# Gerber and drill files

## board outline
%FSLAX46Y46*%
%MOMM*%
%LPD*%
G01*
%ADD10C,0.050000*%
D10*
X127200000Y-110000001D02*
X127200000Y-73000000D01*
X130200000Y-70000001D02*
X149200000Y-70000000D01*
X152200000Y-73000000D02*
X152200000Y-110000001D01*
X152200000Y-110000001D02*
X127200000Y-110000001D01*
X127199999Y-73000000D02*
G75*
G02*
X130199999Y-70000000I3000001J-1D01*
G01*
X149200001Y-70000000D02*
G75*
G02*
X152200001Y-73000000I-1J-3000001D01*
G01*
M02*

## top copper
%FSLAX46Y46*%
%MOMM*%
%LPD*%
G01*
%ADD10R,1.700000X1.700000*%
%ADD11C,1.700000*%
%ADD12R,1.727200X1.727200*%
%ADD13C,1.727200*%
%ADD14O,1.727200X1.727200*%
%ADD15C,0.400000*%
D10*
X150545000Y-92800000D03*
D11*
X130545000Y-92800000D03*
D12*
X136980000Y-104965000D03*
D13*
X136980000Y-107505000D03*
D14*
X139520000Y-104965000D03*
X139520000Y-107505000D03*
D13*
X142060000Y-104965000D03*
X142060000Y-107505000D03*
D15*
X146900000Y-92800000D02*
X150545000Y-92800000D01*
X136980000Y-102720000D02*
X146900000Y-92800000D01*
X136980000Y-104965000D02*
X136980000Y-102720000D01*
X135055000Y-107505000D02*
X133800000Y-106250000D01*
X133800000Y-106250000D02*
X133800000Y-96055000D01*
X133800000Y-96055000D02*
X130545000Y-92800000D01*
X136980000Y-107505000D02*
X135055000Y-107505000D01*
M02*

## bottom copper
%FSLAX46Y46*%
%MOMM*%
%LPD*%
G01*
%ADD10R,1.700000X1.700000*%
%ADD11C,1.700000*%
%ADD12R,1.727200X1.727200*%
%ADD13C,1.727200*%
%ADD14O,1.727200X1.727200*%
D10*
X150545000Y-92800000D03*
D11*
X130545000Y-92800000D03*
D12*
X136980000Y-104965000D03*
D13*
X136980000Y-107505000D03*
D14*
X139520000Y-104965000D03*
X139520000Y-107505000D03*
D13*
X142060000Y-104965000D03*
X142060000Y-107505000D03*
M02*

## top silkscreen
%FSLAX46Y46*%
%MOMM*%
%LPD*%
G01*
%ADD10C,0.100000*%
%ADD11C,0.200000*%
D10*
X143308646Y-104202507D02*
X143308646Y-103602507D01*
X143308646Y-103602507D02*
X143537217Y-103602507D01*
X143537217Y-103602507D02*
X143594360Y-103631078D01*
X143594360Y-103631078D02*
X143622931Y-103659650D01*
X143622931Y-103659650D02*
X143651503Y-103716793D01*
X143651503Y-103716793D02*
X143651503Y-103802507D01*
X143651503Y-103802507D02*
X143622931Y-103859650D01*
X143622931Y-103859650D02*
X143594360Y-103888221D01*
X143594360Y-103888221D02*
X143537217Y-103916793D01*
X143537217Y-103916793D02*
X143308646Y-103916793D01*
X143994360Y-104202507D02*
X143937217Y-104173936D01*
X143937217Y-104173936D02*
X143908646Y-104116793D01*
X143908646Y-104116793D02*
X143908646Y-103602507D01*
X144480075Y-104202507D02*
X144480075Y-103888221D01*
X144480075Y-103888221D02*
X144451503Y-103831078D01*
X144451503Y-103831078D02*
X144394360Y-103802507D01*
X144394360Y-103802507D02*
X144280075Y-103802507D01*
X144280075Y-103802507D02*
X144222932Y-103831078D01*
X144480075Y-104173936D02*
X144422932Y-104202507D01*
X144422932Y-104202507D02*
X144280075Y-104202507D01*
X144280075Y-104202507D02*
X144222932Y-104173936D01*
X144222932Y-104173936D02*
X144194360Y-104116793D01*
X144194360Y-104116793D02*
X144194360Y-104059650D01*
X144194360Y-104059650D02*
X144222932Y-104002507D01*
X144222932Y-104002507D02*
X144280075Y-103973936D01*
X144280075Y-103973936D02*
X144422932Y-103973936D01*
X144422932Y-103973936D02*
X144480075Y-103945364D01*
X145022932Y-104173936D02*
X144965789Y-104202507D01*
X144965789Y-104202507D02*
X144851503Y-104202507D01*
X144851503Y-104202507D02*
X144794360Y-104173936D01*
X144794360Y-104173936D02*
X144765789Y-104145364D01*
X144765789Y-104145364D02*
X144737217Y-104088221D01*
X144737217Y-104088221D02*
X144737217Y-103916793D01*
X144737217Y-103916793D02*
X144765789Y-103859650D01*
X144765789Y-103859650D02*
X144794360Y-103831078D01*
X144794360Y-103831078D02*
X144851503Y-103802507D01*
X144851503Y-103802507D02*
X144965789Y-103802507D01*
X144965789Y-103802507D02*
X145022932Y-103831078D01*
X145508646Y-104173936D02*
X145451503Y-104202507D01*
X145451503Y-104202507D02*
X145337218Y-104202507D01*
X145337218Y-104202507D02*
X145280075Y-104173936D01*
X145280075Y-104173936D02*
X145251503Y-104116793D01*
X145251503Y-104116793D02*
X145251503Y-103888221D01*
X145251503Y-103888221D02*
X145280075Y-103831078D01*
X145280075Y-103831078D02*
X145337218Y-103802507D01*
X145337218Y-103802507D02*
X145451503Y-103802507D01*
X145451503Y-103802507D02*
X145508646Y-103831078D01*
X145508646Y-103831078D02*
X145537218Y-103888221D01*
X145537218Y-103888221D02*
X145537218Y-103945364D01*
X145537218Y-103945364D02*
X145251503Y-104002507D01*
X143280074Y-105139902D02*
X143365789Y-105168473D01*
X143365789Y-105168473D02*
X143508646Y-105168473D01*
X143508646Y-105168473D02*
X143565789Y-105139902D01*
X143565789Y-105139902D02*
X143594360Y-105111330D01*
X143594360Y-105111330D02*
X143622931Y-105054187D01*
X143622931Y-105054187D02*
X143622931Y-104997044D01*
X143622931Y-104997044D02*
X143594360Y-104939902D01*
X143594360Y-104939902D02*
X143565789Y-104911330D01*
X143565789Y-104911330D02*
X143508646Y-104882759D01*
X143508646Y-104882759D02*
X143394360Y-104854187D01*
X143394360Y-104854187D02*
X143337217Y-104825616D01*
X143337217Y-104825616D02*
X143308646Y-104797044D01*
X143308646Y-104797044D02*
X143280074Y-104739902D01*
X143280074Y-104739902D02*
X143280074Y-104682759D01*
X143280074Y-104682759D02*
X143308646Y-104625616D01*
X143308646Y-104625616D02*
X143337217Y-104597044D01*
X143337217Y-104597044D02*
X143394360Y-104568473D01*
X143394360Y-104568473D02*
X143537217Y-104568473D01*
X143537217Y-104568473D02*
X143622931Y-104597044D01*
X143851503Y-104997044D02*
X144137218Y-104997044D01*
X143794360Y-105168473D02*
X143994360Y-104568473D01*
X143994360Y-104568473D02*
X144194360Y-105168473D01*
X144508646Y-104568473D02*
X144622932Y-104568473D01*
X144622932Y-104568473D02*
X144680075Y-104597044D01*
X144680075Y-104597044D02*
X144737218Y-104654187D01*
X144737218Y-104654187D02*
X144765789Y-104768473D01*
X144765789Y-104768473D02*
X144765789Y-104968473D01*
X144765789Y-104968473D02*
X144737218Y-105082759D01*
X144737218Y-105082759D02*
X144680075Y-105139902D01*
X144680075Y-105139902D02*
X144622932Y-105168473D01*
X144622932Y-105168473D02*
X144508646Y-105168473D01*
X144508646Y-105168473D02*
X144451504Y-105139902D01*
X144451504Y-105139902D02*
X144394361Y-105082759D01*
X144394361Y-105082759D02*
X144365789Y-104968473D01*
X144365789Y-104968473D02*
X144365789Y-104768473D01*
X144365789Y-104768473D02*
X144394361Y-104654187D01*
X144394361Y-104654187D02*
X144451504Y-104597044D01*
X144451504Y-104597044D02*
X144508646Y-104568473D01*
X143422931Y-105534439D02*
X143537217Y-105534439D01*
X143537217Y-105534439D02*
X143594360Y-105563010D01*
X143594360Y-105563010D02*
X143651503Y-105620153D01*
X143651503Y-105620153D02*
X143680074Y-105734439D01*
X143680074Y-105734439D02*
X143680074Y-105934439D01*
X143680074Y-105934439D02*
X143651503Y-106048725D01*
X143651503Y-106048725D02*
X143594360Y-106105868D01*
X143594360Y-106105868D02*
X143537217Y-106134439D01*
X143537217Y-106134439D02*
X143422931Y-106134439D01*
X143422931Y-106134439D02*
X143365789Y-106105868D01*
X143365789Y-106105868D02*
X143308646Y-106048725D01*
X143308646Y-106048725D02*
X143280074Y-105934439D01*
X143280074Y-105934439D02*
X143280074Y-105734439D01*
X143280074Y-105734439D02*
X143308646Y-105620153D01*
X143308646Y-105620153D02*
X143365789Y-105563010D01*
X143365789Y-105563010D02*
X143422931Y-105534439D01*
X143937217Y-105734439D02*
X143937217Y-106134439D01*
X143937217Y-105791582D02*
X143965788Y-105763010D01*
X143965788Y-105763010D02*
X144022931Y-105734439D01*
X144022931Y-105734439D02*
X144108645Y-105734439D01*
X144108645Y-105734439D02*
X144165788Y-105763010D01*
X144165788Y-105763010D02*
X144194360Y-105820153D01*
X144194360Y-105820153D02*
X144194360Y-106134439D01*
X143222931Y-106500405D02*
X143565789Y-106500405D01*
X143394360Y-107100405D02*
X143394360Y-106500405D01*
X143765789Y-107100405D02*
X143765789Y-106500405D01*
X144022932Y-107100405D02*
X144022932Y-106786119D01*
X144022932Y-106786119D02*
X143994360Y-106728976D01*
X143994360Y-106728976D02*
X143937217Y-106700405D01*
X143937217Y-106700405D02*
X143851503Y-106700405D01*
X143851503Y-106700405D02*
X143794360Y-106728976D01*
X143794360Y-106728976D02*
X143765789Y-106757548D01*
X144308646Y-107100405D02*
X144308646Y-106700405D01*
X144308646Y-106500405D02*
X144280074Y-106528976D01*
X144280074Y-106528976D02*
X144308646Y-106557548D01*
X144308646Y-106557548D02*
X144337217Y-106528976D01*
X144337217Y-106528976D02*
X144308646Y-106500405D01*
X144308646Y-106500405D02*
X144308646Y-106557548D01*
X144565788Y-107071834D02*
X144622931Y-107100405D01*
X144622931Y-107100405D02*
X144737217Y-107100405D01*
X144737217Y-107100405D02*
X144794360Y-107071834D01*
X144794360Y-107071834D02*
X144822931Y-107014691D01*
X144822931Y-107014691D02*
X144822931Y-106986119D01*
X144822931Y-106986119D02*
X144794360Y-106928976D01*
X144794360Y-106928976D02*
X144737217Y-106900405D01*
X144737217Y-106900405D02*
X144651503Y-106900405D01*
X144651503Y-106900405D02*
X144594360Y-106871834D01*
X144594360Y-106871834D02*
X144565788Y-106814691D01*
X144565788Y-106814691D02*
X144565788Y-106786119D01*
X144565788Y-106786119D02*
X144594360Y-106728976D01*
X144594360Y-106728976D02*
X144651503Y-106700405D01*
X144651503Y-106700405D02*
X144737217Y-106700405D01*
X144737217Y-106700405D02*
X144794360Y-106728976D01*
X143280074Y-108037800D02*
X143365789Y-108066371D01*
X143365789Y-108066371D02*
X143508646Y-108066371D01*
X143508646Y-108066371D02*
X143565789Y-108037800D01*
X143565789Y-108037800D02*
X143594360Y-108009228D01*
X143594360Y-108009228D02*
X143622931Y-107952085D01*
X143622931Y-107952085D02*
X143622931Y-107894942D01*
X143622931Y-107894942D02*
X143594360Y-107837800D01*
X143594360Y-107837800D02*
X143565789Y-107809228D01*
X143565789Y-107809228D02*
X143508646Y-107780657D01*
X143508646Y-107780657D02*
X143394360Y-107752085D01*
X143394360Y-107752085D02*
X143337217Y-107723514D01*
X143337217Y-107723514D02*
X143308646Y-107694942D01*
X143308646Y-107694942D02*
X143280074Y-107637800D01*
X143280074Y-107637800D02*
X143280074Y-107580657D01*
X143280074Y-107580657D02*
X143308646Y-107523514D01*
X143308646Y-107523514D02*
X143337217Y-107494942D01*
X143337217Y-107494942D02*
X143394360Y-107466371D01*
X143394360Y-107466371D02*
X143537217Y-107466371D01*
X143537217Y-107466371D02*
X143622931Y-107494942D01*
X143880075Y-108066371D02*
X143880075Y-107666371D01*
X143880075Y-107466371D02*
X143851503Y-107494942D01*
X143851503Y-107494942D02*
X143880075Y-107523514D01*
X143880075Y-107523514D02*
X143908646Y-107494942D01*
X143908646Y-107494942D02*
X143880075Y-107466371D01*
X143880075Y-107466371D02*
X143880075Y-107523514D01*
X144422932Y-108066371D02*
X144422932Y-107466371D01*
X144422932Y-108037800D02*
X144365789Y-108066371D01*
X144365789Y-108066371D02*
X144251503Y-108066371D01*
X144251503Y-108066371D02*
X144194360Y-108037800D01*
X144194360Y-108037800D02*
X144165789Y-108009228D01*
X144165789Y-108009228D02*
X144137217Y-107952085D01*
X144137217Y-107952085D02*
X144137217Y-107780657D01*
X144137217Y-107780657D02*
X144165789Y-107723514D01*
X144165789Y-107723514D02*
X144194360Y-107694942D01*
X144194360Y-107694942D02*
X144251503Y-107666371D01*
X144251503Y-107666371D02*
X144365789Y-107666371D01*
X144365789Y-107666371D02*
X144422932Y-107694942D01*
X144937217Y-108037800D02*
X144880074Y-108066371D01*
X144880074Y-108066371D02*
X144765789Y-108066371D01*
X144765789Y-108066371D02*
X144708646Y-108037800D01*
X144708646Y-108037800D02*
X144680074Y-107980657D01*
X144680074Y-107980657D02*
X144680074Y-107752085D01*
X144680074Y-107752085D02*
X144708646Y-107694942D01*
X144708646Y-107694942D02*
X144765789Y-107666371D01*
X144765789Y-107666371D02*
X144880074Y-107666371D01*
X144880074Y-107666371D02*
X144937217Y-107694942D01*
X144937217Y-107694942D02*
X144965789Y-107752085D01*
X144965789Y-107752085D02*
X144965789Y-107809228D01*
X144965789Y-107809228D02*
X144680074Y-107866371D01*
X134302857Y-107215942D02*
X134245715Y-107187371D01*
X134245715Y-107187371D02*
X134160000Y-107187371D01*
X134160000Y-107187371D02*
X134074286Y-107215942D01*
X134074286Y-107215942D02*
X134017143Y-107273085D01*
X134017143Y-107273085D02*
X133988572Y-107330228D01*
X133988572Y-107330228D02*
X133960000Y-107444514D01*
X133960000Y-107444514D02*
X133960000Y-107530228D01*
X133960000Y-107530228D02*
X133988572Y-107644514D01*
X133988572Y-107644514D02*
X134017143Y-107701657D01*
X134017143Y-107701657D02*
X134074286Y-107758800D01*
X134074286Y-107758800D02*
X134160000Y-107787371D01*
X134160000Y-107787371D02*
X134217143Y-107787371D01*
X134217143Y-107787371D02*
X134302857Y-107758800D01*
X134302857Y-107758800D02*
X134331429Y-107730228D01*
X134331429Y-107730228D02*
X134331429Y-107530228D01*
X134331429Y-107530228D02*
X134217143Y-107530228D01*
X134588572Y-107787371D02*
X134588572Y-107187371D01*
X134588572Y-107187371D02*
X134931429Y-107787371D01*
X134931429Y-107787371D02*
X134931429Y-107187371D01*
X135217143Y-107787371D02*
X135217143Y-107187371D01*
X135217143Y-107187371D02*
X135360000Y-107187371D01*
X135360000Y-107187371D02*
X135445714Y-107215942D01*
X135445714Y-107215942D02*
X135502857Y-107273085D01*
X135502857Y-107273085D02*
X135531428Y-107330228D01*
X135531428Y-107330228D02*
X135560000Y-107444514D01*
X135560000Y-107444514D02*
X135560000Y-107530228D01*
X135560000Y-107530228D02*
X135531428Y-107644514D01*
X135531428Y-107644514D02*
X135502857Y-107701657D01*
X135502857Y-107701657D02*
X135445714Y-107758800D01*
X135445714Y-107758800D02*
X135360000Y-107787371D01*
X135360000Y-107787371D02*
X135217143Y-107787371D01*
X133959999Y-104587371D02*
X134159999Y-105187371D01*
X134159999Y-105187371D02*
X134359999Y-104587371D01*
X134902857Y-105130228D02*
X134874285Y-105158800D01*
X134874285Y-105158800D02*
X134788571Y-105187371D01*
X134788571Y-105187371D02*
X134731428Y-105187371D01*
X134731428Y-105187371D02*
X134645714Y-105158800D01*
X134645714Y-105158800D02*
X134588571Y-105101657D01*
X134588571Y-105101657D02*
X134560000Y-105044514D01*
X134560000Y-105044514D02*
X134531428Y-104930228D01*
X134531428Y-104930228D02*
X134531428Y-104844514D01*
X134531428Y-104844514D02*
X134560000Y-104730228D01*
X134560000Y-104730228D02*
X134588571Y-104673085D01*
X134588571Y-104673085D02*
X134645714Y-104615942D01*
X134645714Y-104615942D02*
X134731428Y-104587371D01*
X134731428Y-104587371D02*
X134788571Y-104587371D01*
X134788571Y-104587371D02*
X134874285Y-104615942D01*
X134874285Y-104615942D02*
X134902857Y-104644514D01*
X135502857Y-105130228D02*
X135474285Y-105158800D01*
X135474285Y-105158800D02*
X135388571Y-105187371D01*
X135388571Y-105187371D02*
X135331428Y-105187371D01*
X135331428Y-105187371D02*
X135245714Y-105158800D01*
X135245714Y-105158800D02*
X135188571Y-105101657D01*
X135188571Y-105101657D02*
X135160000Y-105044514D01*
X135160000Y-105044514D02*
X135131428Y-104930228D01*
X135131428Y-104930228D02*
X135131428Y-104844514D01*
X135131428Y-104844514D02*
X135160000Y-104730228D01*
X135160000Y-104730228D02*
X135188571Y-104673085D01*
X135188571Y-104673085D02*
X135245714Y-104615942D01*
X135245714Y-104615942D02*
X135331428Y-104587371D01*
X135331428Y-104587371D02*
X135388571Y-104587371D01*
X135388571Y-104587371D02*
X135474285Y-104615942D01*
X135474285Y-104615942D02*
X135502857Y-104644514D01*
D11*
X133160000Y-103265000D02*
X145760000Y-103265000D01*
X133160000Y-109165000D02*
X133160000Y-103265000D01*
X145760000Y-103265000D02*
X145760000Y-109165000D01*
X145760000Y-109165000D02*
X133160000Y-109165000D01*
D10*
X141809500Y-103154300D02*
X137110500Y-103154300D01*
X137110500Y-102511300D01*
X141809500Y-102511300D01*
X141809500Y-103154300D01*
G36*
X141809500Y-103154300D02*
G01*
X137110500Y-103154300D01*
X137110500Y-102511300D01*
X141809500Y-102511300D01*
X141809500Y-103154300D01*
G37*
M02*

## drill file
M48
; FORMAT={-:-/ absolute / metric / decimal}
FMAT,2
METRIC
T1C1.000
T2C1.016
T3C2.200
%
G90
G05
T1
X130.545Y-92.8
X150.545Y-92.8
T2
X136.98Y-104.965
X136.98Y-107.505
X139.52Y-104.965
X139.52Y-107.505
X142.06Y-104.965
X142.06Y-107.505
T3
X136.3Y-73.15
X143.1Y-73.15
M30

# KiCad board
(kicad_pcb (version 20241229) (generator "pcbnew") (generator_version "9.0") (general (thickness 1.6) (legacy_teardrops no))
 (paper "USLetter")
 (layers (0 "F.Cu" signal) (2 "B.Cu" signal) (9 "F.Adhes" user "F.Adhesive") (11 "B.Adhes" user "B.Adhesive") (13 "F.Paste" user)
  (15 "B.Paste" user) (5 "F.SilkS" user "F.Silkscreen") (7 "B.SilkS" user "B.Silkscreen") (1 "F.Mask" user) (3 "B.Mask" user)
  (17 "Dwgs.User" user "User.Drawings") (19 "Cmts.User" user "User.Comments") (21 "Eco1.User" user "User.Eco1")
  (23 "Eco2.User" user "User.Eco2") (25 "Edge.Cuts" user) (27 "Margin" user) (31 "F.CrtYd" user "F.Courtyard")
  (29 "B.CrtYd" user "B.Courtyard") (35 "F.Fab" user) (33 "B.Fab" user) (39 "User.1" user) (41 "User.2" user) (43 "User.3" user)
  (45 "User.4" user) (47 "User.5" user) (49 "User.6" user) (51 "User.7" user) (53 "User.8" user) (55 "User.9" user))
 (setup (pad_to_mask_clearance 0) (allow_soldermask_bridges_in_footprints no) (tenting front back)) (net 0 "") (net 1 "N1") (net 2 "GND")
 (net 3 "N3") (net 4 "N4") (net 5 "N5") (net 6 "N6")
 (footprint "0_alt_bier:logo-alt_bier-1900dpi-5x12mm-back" (layer "F.Cu") (at 149.510685 81.365872)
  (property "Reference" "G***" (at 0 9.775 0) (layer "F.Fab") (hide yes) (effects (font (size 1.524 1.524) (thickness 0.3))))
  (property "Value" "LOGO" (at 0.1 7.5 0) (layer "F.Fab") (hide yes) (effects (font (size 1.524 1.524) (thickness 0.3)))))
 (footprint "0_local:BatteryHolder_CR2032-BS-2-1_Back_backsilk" (layer "F.Cu") (at 127.545 92.8 90)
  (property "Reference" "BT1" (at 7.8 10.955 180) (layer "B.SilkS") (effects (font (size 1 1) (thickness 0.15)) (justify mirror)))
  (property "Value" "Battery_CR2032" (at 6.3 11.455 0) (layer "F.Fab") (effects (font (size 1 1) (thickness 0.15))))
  (pad "1" thru_hole rect (at 0 23 90) (size 1.7 1.7) (drill 1) (layers "*.Cu" "*.Mask") (remove_unused_layers no) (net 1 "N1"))
  (pad "2" thru_hole circle (at 0 3 90) (size 1.7 1.7) (drill 1) (layers "*.Cu" "*.Mask") (remove_unused_layers no) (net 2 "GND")))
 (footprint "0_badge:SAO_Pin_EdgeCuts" (layer "F.Cu") (at 139.7 88.000001)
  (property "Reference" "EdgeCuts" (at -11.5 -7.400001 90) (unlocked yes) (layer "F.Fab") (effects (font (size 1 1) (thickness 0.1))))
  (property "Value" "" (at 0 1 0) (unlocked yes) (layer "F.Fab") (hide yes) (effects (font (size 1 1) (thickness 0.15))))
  (fp_line (start -12.5 22) (end -12.5 -15.000001) (stroke (width 0.05) (type default)) (layer "Edge.Cuts"))
  (fp_line (start -9.5 -18) (end 9.5 -18.000001) (stroke (width 0.05) (type default)) (layer "Edge.Cuts"))
  (fp_line (start 12.5 -15.000001) (end 12.5 22) (stroke (width 0.05) (type default)) (layer "Edge.Cuts"))
  (fp_line (start 12.5 22) (end -12.5 22) (stroke (width 0.05) (type default)) (layer "Edge.Cuts"))
  (fp_arc (start -12.500001 -15.000001) (mid -11.621321 -17.121321) (end -9.500001 -18.000001) (stroke (width 0.05) (type default))
   (layer "Edge.Cuts"))
  (fp_arc (start 9.500001 -18.000001) (mid 11.621321 -17.121321) (end 12.500001 -15.000001) (stroke (width 0.05) (type default))
   (layer "Edge.Cuts")))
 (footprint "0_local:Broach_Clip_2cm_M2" (layer "F.Cu") (at 139.7 73.15)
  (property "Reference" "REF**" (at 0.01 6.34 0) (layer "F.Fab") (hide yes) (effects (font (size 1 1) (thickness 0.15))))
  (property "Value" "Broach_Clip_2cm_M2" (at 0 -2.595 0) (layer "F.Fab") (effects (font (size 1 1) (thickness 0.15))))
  (pad "" np_thru_hole circle (at -3.4 0) (size 2.2 2.2) (drill 2.2) (layers "*.Cu" "*.Mask"))
  (pad "" np_thru_hole circle (at 3.4 0) (size 2.2 2.2) (drill 2.2) (layers "*.Cu" "*.Mask")))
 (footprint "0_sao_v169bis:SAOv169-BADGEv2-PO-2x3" (layer "F.Cu") (at 139.46 106.215)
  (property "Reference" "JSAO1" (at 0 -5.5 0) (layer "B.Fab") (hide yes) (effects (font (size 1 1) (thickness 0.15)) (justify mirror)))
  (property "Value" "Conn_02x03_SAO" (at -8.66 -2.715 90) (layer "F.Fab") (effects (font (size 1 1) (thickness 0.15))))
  (fp_line (start -6.3 -2.95) (end 6.3 -2.95) (stroke (width 0.2) (type solid)) (layer "F.SilkS"))
  (fp_line (start -6.3 2.95) (end -6.3 -2.95) (stroke (width 0.2) (type solid)) (layer "F.SilkS"))
  (fp_line (start 6.3 -2.95) (end 6.3 2.95) (stroke (width 0.2) (type solid)) (layer "F.SilkS"))
  (fp_line (start 6.3 2.95) (end -6.3 2.95) (stroke (width 0.2) (type solid)) (layer "F.SilkS"))
  (fp_poly
   (pts (xy 2.3495 -3.0607) (xy -2.3495 -3.0607) (xy -2.3495 -3.7037) (xy 2.3495 -3.7037)) (stroke (width 0.1) (type solid)) (fill yes)
   (layer "F.SilkS"))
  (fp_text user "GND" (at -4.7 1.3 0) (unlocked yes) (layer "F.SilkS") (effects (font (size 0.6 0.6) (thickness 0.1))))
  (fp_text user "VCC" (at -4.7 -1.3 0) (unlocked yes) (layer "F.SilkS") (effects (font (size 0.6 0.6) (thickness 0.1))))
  (pad "1" thru_hole rect (at -2.48 -1.25 270) (size 1.7272 1.7272) (drill 1.016) (layers "*.Cu" "*.Mask") (remove_unused_layers no)
   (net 1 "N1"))
  (pad "2" thru_hole circle (at -2.48 1.29 270) (size 1.7272 1.7272) (drill 1.016) (layers "*.Cu" "*.Mask") (remove_unused_layers no)
   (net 2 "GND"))
  (pad "3" thru_hole oval (at 0.06 -1.25 270) (size 1.7272 1.7272) (drill 1.016) (layers "*.Cu" "*.Mask") (remove_unused_layers no)
   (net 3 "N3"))
  (pad "4" thru_hole oval (at 0.06 1.29 270) (size 1.7272 1.7272) (drill 1.016) (layers "*.Cu" "*.Mask") (remove_unused_layers no)
   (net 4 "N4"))
  (pad "5" thru_hole circle (at 2.6 -1.25 270) (size 1.7272 1.7272) (drill 1.016) (layers "*.Cu" "*.Mask") (remove_unused_layers no)
   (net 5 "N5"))
  (pad "6" thru_hole circle (at 2.6 1.29 270) (size 1.7272 1.7272) (drill 1.016) (layers "*.Cu" "*.Mask") (remove_unused_layers no)
   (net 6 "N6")))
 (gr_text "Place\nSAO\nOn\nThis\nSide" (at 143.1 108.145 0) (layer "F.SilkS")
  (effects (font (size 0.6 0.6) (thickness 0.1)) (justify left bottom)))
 (segment (start 146.9 92.8) (end 150.545 92.8) (width 0.4) (layer "F.Cu") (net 1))
 (segment (start 136.98 102.72) (end 146.9 92.8) (width 0.4) (layer "F.Cu") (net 1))
 (segment (start 136.98 104.965) (end 136.98 102.72) (width 0.4) (layer "F.Cu") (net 1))
 (segment (start 135.055 107.505) (end 133.8 106.25) (width 0.4) (layer "F.Cu") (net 2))
 (segment (start 133.8 106.25) (end 133.8 96.055) (width 0.4) (layer "F.Cu") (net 2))
 (segment (start 133.8 96.055) (end 130.545 92.8) (width 0.4) (layer "F.Cu") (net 2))
 (segment (start 136.98 107.505) (end 135.055 107.505) (width 0.4) (layer "F.Cu") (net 2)))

